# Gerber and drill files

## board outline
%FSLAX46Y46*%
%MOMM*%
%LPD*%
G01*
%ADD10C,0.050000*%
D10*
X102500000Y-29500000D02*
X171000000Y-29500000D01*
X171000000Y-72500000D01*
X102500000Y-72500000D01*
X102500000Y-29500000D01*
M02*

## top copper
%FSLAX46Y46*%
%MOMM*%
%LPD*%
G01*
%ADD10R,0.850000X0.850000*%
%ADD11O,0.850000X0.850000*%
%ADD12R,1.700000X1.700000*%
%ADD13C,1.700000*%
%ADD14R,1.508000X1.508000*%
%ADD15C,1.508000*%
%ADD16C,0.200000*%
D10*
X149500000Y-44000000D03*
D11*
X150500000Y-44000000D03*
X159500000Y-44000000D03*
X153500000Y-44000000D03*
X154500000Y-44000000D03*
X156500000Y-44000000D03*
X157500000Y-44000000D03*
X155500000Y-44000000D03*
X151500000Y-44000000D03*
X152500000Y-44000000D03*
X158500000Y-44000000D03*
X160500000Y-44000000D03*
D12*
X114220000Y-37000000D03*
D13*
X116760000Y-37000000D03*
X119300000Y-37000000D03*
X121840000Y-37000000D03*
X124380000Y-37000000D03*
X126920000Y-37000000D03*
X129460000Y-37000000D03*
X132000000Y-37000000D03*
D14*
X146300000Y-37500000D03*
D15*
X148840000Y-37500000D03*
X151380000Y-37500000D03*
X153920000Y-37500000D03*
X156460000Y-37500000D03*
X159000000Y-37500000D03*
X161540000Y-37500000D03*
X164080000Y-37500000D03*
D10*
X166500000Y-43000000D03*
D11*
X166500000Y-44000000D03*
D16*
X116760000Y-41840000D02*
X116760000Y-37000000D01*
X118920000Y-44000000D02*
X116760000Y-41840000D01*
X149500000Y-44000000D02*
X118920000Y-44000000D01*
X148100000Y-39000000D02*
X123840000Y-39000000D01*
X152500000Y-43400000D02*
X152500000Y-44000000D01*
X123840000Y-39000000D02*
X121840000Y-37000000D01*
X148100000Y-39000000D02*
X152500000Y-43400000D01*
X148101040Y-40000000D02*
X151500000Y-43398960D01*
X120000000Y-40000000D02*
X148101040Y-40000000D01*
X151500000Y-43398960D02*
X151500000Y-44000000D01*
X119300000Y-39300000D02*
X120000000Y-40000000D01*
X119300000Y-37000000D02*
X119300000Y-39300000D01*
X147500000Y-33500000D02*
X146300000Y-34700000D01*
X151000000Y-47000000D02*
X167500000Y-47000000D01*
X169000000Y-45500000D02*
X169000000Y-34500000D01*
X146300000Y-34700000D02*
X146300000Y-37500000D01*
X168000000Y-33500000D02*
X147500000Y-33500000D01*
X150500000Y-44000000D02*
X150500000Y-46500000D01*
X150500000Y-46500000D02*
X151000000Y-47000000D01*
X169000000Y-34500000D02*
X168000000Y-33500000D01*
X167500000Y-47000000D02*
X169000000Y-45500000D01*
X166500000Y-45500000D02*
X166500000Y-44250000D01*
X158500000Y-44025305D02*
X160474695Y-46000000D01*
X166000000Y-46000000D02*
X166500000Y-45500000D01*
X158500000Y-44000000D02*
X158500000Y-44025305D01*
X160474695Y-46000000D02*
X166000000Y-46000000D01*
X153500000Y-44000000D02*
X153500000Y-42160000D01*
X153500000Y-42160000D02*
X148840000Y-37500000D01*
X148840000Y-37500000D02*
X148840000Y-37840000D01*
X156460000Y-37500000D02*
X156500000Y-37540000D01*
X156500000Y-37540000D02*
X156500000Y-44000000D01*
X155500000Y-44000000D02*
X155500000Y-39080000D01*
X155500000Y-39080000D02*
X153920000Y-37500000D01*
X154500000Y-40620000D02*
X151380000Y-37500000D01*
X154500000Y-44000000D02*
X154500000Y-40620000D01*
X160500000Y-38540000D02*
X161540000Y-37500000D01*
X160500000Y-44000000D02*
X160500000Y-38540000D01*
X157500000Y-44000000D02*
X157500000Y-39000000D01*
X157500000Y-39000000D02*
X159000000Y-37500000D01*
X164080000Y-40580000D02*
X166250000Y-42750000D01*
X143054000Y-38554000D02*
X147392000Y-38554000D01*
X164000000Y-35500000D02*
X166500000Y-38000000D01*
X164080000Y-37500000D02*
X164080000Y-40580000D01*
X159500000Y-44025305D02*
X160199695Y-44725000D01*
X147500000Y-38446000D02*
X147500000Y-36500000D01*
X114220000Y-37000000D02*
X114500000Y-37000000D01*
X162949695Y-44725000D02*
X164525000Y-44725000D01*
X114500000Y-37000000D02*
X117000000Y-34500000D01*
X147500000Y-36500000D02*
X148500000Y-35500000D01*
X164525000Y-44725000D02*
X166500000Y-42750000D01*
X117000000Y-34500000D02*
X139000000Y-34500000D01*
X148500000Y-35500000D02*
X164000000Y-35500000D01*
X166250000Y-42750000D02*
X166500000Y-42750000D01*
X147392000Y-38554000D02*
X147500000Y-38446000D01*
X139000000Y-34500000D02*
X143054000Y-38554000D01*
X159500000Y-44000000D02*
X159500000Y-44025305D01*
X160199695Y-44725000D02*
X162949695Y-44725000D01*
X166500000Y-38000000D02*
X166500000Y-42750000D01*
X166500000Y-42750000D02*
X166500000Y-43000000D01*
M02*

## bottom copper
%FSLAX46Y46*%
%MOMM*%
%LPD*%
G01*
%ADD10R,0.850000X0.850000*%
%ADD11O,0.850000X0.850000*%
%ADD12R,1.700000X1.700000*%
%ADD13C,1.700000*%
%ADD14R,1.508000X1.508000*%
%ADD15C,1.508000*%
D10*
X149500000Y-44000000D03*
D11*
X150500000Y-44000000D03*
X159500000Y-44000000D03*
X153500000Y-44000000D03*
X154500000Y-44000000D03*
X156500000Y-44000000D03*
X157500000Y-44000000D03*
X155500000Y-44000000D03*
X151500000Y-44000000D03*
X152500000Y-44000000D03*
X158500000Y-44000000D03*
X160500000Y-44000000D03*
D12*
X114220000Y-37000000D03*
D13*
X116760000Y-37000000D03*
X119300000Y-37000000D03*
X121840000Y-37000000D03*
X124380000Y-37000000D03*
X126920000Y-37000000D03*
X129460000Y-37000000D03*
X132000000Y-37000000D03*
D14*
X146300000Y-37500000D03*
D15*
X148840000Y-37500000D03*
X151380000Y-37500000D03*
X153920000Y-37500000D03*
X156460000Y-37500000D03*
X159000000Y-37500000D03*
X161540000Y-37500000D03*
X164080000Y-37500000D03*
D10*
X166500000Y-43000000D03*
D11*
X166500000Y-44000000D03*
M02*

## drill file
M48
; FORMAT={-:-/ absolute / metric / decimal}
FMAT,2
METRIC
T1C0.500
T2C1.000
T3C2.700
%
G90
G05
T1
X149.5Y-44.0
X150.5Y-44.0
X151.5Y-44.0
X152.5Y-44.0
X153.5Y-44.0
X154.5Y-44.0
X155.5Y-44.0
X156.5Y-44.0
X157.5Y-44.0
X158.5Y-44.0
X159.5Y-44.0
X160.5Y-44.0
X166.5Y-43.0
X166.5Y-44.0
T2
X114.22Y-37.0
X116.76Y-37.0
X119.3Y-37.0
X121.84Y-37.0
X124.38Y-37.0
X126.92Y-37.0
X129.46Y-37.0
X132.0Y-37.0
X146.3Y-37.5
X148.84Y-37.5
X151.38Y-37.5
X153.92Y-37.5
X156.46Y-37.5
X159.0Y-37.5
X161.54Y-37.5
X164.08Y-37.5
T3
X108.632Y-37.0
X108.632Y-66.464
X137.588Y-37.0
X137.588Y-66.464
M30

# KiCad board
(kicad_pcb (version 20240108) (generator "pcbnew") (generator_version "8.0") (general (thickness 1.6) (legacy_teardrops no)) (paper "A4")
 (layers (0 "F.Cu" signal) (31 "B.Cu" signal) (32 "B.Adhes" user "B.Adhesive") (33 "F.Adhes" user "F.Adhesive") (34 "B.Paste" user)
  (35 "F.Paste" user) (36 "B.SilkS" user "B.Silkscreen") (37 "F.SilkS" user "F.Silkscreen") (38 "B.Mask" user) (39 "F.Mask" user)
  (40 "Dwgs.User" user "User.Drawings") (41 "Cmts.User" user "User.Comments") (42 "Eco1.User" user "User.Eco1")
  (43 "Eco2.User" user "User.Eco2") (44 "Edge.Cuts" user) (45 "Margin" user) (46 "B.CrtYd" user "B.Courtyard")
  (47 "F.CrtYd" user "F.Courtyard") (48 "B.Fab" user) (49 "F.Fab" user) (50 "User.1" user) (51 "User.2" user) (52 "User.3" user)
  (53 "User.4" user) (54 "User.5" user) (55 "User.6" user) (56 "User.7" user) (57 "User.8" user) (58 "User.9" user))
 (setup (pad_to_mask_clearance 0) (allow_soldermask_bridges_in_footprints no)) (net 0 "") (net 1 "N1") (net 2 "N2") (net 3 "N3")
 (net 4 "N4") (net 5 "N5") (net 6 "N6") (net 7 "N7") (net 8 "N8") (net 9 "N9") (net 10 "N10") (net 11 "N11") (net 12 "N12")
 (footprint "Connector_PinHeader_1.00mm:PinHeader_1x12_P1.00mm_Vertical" (layer "F.Cu") (at 149.5 44 90)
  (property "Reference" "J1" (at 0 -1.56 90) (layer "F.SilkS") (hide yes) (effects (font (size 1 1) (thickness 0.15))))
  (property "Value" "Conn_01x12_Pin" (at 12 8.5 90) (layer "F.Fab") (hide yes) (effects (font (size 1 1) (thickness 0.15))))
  (pad "1" thru_hole rect (at 0 0 90) (size 0.85 0.85) (drill 0.5) (layers "*.Cu" "*.Mask") (remove_unused_layers no) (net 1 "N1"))
  (pad "2" thru_hole oval (at 0 1 90) (size 0.85 0.85) (drill 0.5) (layers "*.Cu" "*.Mask") (remove_unused_layers no) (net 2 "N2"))
  (pad "3" thru_hole oval (at 0 10 90) (size 0.85 0.85) (drill 0.5) (layers "*.Cu" "*.Mask") (remove_unused_layers no) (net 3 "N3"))
  (pad "4" thru_hole oval (at 0 4 90) (size 0.85 0.85) (drill 0.5) (layers "*.Cu" "*.Mask") (remove_unused_layers no) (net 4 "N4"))
  (pad "5" thru_hole oval (at 0 5 90) (size 0.85 0.85) (drill 0.5) (layers "*.Cu" "*.Mask") (remove_unused_layers no) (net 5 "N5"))
  (pad "6" thru_hole oval (at 0 7 90) (size 0.85 0.85) (drill 0.5) (layers "*.Cu" "*.Mask") (remove_unused_layers no) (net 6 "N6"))
  (pad "7" thru_hole oval (at 0 8 90) (size 0.85 0.85) (drill 0.5) (layers "*.Cu" "*.Mask") (remove_unused_layers no) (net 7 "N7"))
  (pad "8" thru_hole oval (at 0 6 90) (size 0.85 0.85) (drill 0.5) (layers "*.Cu" "*.Mask") (remove_unused_layers no) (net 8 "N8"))
  (pad "9" thru_hole oval (at 0 2 90) (size 0.85 0.85) (drill 0.5) (layers "*.Cu" "*.Mask") (remove_unused_layers no) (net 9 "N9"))
  (pad "10" thru_hole oval (at 0 3 90) (size 0.85 0.85) (drill 0.5) (layers "*.Cu" "*.Mask") (remove_unused_layers no) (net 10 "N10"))
  (pad "11" thru_hole oval (at 0 9 90) (size 0.85 0.85) (drill 0.5) (layers "*.Cu" "*.Mask") (remove_unused_layers no) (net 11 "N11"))
  (pad "12" thru_hole oval (at 0 11 90) (size 0.85 0.85) (drill 0.5) (layers "*.Cu" "*.Mask") (remove_unused_layers no) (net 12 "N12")))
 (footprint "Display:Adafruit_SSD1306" (layer "F.Cu") (at 114.22 37)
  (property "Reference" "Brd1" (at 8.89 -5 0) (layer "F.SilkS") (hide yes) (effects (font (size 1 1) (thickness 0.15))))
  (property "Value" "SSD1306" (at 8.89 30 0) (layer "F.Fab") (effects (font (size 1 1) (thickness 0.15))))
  (pad "" np_thru_hole circle (at -5.588 0) (size 2.7 2.7) (drill 2.7) (layers "*.Cu" "*.Mask"))
  (pad "" np_thru_hole circle (at -5.588 29.464) (size 2.7 2.7) (drill 2.7) (layers "*.Cu" "*.Mask"))
  (pad "" np_thru_hole circle (at 23.368 0) (size 2.7 2.7) (drill 2.7) (layers "*.Cu" "*.Mask"))
  (pad "" np_thru_hole circle (at 23.368 29.464) (size 2.7 2.7) (drill 2.7) (layers "*.Cu" "*.Mask"))
  (pad "1" thru_hole rect (at 0 0) (size 1.7 1.7) (drill 1) (layers "*.Cu" "*.Mask") (remove_unused_layers no) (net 3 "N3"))
  (pad "2" thru_hole circle (at 2.54 0) (size 1.7 1.7) (drill 1) (layers "*.Cu" "*.Mask") (remove_unused_layers no) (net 1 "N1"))
  (pad "3" thru_hole circle (at 5.08 0) (size 1.7 1.7) (drill 1) (layers "*.Cu" "*.Mask") (remove_unused_layers no) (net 9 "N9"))
  (pad "4" thru_hole circle (at 7.62 0) (size 1.7 1.7) (drill 1) (layers "*.Cu" "*.Mask") (remove_unused_layers no) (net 10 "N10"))
  (pad "5" thru_hole circle (at 10.16 0) (size 1.7 1.7) (drill 1) (layers "*.Cu" "*.Mask") (remove_unused_layers no))
  (pad "6" thru_hole circle (at 12.7 0) (size 1.7 1.7) (drill 1) (layers "*.Cu" "*.Mask") (remove_unused_layers no))
  (pad "7" thru_hole circle (at 15.24 0) (size 1.7 1.7) (drill 1) (layers "*.Cu" "*.Mask") (remove_unused_layers no))
  (pad "8" thru_hole circle (at 17.78 0) (size 1.7 1.7) (drill 1) (layers "*.Cu" "*.Mask") (remove_unused_layers no)))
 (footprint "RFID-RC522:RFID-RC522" (layer "F.Cu") (at 155.19 37.5)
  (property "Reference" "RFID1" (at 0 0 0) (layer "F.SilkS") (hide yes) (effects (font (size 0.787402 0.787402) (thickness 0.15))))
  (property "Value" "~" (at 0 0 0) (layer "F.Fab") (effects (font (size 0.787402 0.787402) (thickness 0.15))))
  (pad "1" thru_hole rect (at -8.89 0) (size 1.508 1.508) (drill 1) (layers "*.Cu" "*.Mask") (remove_unused_layers no) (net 2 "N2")
   (solder_mask_margin 0.102))
  (pad "2" thru_hole circle (at -6.35 0) (size 1.508 1.508) (drill 1) (layers "*.Cu" "*.Mask") (remove_unused_layers no) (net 4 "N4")
   (solder_mask_margin 0.102))
  (pad "3" thru_hole circle (at -3.81 0) (size 1.508 1.508) (drill 1) (layers "*.Cu" "*.Mask") (remove_unused_layers no) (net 5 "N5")
   (solder_mask_margin 0.102))
  (pad "4" thru_hole circle (at -1.27 0) (size 1.508 1.508) (drill 1) (layers "*.Cu" "*.Mask") (remove_unused_layers no) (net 8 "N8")
   (solder_mask_margin 0.102))
  (pad "5" thru_hole circle (at 1.27 0) (size 1.508 1.508) (drill 1) (layers "*.Cu" "*.Mask") (remove_unused_layers no) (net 6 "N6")
   (solder_mask_margin 0.102))
  (pad "6" thru_hole circle (at 3.81 0) (size 1.508 1.508) (drill 1) (layers "*.Cu" "*.Mask") (remove_unused_layers no) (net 7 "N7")
   (solder_mask_margin 0.102))
  (pad "7" thru_hole circle (at 6.35 0) (size 1.508 1.508) (drill 1) (layers "*.Cu" "*.Mask") (remove_unused_layers no) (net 12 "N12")
   (solder_mask_margin 0.102))
  (pad "8" thru_hole circle (at 8.89 0) (size 1.508 1.508) (drill 1) (layers "*.Cu" "*.Mask") (remove_unused_layers no) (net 3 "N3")
   (solder_mask_margin 0.102)))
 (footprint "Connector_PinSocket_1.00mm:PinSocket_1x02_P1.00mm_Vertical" (layer "F.Cu") (at 166.5 43)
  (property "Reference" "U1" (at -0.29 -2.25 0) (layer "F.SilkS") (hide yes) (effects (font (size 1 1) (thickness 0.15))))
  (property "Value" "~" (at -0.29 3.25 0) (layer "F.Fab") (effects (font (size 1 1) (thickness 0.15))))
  (pad "1" thru_hole rect (at 0 0) (size 0.85 0.85) (drill 0.5) (layers "*.Cu" "*.Mask") (remove_unused_layers no) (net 3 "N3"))
  (pad "2" thru_hole oval (at 0 1) (size 0.85 0.85) (drill 0.5) (layers "*.Cu" "*.Mask") (remove_unused_layers no) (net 11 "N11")))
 (gr_rect (start 102.5 29.5) (end 171 72.5) (stroke (width 0.05) (type default)) (fill none) (layer "Edge.Cuts"))
 (segment (start 116.76 41.84) (end 116.76 37) (width 0.2) (layer "F.Cu") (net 1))
 (segment (start 118.92 44) (end 116.76 41.84) (width 0.2) (layer "F.Cu") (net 1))
 (segment (start 149.5 44) (end 118.92 44) (width 0.2) (layer "F.Cu") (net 1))
 (segment (start 148.1 39) (end 123.84 39) (width 0.2) (layer "F.Cu") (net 10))
 (segment (start 152.5 43.4) (end 152.5 44) (width 0.2) (layer "F.Cu") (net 10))
 (segment (start 123.84 39) (end 121.84 37) (width 0.2) (layer "F.Cu") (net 10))
 (segment (start 148.1 39) (end 152.5 43.4) (width 0.2) (layer "F.Cu") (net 10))
 (segment (start 148.10104 40) (end 151.5 43.39896) (width 0.2) (layer "F.Cu") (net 9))
 (segment (start 120 40) (end 148.10104 40) (width 0.2) (layer "F.Cu") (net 9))
 (segment (start 151.5 43.39896) (end 151.5 44) (width 0.2) (layer "F.Cu") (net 9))
 (segment (start 119.3 39.3) (end 120 40) (width 0.2) (layer "F.Cu") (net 9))
 (segment (start 119.3 37) (end 119.3 39.3) (width 0.2) (layer "F.Cu") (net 9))
 (segment (start 147.5 33.5) (end 146.3 34.7) (width 0.2) (layer "F.Cu") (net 2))
 (segment (start 151 47) (end 167.5 47) (width 0.2) (layer "F.Cu") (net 2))
 (segment (start 169 45.5) (end 169 34.5) (width 0.2) (layer "F.Cu") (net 2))
 (segment (start 146.3 34.7) (end 146.3 37.5) (width 0.2) (layer "F.Cu") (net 2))
 (segment (start 168 33.5) (end 147.5 33.5) (width 0.2) (layer "F.Cu") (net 2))
 (segment (start 150.5 44) (end 150.5 46.5) (width 0.2) (layer "F.Cu") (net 2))
 (segment (start 150.5 46.5) (end 151 47) (width 0.2) (layer "F.Cu") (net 2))
 (segment (start 169 34.5) (end 168 33.5) (width 0.2) (layer "F.Cu") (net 2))
 (segment (start 167.5 47) (end 169 45.5) (width 0.2) (layer "F.Cu") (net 2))
 (segment (start 166.5 45.5) (end 166.5 44.25) (width 0.2) (layer "F.Cu") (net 11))
 (segment (start 158.5 44.025305) (end 160.474695 46) (width 0.2) (layer "F.Cu") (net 11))
 (segment (start 166 46) (end 166.5 45.5) (width 0.2) (layer "F.Cu") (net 11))
 (segment (start 158.5 44) (end 158.5 44.025305) (width 0.2) (layer "F.Cu") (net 11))
 (segment (start 160.474695 46) (end 166 46) (width 0.2) (layer "F.Cu") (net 11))
 (segment (start 153.5 44) (end 153.5 42.16) (width 0.2) (layer "F.Cu") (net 4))
 (segment (start 153.5 42.16) (end 148.84 37.5) (width 0.2) (layer "F.Cu") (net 4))
 (segment (start 148.84 37.5) (end 148.84 37.84) (width 0.2) (layer "F.Cu") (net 4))
 (segment (start 156.46 37.5) (end 156.5 37.54) (width 0.2) (layer "F.Cu") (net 6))
 (segment (start 156.5 37.54) (end 156.5 44) (width 0.2) (layer "F.Cu") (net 6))
 (segment (start 155.5 44) (end 155.5 39.08) (width 0.2) (layer "F.Cu") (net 8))
 (segment (start 155.5 39.08) (end 153.92 37.5) (width 0.2) (layer "F.Cu") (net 8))
 (segment (start 154.5 40.62) (end 151.38 37.5) (width 0.2) (layer "F.Cu") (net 5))
 (segment (start 154.5 44) (end 154.5 40.62) (width 0.2) (layer "F.Cu") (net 5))
 (segment (start 160.5 38.54) (end 161.54 37.5) (width 0.2) (layer "F.Cu") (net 12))
 (segment (start 160.5 44) (end 160.5 38.54) (width 0.2) (layer "F.Cu") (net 12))
 (segment (start 157.5 44) (end 157.5 39) (width 0.2) (layer "F.Cu") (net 7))
 (segment (start 157.5 39) (end 159 37.5) (width 0.2) (layer "F.Cu") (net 7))
 (segment (start 164.08 40.58) (end 166.25 42.75) (width 0.2) (layer "F.Cu") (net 3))
 (segment (start 143.054 38.554) (end 147.392 38.554) (width 0.2) (layer "F.Cu") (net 3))
 (segment (start 164 35.5) (end 166.5 38) (width 0.2) (layer "F.Cu") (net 3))
 (segment (start 164.08 37.5) (end 164.08 40.58) (width 0.2) (layer "F.Cu") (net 3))
 (segment (start 159.5 44.025305) (end 160.199695 44.725) (width 0.2) (layer "F.Cu") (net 3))
 (segment (start 147.5 38.446) (end 147.5 36.5) (width 0.2) (layer "F.Cu") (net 3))
 (segment (start 114.22 37) (end 114.5 37) (width 0.2) (layer "F.Cu") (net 3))
 (segment (start 162.949695 44.725) (end 164.525 44.725) (width 0.2) (layer "F.Cu") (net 3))
 (segment (start 114.5 37) (end 117 34.5) (width 0.2) (layer "F.Cu") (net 3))
 (segment (start 147.5 36.5) (end 148.5 35.5) (width 0.2) (layer "F.Cu") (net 3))
 (segment (start 164.525 44.725) (end 166.5 42.75) (width 0.2) (layer "F.Cu") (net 3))
 (segment (start 117 34.5) (end 139 34.5) (width 0.2) (layer "F.Cu") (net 3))
 (segment (start 148.5 35.5) (end 164 35.5) (width 0.2) (layer "F.Cu") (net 3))
 (segment (start 166.25 42.75) (end 166.5 42.75) (width 0.2) (layer "F.Cu") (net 3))
 (segment (start 147.392 38.554) (end 147.5 38.446) (width 0.2) (layer "F.Cu") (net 3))
 (segment (start 139 34.5) (end 143.054 38.554) (width 0.2) (layer "F.Cu") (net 3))
 (segment (start 159.5 44) (end 159.5 44.025305) (width 0.2) (layer "F.Cu") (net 3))
 (segment (start 160.199695 44.725) (end 162.949695 44.725) (width 0.2) (layer "F.Cu") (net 3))
 (segment (start 166.5 38) (end 166.5 42.75) (width 0.2) (layer "F.Cu") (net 3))
 (segment (start 166.5 42.75) (end 166.5 43) (width 0.2) (layer "F.Cu") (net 3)))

